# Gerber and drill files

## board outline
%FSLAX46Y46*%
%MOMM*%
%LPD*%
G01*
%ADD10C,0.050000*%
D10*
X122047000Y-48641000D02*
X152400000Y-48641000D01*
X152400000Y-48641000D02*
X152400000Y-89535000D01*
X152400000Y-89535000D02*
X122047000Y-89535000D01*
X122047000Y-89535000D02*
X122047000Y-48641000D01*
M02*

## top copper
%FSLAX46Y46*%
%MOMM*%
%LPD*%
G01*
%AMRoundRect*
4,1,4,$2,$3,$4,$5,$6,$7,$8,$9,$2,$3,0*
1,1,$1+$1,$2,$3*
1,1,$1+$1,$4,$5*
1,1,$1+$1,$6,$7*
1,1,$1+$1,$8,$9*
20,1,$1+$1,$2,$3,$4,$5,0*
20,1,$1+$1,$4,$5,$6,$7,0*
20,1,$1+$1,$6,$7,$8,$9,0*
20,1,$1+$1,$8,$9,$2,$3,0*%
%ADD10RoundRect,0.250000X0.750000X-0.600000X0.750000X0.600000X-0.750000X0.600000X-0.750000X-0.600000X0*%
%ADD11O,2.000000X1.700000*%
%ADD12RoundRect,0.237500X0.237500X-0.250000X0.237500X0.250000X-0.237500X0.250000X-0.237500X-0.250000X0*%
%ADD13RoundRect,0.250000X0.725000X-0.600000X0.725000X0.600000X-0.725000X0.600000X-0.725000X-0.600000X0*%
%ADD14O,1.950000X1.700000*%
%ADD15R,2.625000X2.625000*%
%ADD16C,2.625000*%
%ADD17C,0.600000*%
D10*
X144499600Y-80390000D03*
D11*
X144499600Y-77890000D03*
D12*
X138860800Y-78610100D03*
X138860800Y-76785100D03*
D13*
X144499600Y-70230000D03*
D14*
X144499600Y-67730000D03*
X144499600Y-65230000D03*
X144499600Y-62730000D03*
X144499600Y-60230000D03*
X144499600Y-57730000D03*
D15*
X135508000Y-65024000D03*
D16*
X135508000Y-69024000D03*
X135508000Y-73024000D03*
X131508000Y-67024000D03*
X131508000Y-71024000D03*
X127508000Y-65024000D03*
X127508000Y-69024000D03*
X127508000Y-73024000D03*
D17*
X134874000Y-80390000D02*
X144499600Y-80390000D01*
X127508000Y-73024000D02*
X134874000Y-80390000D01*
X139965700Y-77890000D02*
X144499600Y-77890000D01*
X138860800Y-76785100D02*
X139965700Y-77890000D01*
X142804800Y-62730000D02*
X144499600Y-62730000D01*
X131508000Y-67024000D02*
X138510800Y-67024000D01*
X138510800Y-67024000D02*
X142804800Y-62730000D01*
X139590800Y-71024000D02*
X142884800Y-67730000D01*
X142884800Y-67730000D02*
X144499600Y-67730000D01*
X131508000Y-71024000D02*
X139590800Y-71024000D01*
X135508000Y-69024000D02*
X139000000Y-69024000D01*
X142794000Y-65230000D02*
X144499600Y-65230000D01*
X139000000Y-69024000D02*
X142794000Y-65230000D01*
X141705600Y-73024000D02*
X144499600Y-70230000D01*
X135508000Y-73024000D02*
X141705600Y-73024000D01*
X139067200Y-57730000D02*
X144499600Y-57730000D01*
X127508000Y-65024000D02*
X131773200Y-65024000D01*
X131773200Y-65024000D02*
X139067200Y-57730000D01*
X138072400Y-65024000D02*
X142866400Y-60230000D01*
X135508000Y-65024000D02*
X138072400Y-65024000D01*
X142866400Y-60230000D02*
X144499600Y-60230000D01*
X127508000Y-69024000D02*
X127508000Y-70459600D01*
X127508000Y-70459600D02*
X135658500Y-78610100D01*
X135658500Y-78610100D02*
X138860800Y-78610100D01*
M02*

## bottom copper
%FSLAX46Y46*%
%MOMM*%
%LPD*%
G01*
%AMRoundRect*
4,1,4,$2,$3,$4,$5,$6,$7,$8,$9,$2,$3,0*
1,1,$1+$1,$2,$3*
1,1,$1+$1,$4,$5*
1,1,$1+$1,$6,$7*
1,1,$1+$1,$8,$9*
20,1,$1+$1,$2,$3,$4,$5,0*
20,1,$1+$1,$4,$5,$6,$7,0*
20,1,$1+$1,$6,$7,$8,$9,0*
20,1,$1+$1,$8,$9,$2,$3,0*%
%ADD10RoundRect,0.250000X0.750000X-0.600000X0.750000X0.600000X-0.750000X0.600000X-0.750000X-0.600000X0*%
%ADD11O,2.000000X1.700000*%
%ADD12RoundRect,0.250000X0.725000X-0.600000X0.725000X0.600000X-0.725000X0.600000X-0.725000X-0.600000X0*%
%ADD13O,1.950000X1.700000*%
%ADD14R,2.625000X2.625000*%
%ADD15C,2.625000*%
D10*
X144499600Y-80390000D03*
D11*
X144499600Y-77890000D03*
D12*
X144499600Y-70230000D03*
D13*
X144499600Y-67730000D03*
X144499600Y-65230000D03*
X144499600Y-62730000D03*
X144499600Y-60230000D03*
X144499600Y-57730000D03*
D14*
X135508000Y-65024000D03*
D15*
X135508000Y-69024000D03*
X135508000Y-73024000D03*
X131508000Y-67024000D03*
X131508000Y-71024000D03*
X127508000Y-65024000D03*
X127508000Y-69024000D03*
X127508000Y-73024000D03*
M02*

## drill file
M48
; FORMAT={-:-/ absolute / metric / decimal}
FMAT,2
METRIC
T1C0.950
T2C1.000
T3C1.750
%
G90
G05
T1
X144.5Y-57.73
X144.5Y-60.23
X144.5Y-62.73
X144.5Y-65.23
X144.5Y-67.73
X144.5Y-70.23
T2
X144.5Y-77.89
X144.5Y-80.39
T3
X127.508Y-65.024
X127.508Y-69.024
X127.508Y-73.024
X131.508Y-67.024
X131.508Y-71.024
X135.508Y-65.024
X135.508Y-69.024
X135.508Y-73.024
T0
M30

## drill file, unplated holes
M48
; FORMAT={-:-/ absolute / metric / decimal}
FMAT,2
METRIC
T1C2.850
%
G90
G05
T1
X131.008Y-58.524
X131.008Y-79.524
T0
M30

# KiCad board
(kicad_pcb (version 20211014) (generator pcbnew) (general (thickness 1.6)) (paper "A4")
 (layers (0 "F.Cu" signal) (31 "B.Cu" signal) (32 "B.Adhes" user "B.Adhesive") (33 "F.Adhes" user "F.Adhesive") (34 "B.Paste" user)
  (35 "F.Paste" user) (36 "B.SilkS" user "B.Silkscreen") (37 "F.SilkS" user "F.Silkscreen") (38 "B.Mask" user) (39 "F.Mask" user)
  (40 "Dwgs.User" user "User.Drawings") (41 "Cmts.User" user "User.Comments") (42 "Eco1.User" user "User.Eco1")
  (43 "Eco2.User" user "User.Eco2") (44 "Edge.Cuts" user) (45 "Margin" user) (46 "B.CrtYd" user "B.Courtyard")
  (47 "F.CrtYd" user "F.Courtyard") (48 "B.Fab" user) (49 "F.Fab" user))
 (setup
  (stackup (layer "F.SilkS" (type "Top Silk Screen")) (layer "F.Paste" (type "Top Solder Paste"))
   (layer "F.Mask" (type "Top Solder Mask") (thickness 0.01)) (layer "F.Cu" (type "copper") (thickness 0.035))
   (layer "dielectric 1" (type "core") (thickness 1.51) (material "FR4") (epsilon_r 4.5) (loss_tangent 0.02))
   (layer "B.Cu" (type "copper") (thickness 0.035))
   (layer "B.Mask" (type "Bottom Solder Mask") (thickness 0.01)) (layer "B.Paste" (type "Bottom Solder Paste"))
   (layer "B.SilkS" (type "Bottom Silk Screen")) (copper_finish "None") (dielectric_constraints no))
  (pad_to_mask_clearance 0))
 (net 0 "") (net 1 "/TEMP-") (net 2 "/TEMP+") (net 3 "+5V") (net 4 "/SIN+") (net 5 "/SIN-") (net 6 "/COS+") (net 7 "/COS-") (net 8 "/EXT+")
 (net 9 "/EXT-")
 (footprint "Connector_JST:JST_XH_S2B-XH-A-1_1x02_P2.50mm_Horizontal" (layer "F.Cu") (at 144.4996 80.39 90)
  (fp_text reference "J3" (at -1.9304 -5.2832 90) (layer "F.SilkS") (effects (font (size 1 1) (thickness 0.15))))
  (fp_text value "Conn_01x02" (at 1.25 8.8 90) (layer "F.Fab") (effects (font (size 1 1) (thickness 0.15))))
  (pad "1" thru_hole roundrect (at 0 0 90) (size 1.7 2) (drill 1) (layers *.Cu *.Mask) (roundrect_rratio 0.1470588235) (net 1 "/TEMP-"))
  (pad "2" thru_hole oval (at 2.5 0 90) (size 1.7 2) (drill 1) (layers *.Cu *.Mask) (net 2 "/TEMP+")))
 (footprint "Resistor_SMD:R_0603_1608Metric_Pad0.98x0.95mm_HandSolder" (layer "F.Cu") (at 138.8608 77.6976 90)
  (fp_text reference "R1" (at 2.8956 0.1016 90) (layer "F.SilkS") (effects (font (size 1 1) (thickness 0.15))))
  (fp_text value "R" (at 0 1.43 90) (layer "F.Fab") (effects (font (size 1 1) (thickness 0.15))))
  (pad "1" smd roundrect (at -0.9125 0 90) (size 0.975 0.95) (layers "F.Cu" "F.Paste" "F.Mask") (roundrect_rratio 0.25) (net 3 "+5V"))
  (pad "2" smd roundrect (at 0.9125 0 90) (size 0.975 0.95) (layers "F.Cu" "F.Paste" "F.Mask") (roundrect_rratio 0.25) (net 2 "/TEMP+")))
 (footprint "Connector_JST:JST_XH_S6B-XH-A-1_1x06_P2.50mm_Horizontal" (layer "F.Cu") (at 144.4996 70.23 90)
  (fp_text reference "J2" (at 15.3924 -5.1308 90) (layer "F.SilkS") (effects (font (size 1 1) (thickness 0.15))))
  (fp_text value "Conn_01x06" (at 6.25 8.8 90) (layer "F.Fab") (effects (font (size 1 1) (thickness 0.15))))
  (pad "1" thru_hole roundrect (at 0 0 90) (size 1.7 1.95) (drill 0.95) (layers *.Cu *.Mask) (roundrect_rratio 0.1470588235) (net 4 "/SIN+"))
  (pad "2" thru_hole oval (at 2.5 0 90) (size 1.7 1.95) (drill 0.95) (layers *.Cu *.Mask) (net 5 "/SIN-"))
  (pad "3" thru_hole oval (at 5 0 90) (size 1.7 1.95) (drill 0.95) (layers *.Cu *.Mask) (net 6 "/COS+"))
  (pad "4" thru_hole oval (at 7.5 0 90) (size 1.7 1.95) (drill 0.95) (layers *.Cu *.Mask) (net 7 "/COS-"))
  (pad "5" thru_hole oval (at 10 0 90) (size 1.7 1.95) (drill 0.95) (layers *.Cu *.Mask) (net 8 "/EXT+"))
  (pad "6" thru_hole oval (at 12.5 0 90) (size 1.7 1.95) (drill 0.95) (layers *.Cu *.Mask) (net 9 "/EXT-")))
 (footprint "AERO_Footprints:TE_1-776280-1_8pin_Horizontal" (layer "F.Cu") (at 131.008 69.024 -90)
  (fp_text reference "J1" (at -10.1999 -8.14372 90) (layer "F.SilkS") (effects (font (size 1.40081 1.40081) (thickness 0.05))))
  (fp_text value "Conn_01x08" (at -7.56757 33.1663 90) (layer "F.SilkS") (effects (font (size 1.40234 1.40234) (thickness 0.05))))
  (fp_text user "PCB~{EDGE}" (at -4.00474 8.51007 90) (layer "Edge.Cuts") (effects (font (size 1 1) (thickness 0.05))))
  (pad "" np_thru_hole circle (at -10.5 0 270) (size 2.85 2.85) (drill 2.85) (layers *.Cu *.Mask "F.SilkS"))
  (pad "" np_thru_hole circle (at 10.5 0 270) (size 2.85 2.85) (drill 2.85) (layers *.Cu *.Mask "F.SilkS"))
  (pad "1" thru_hole rect (at -4 -4.5 270) (size 2.625 2.625) (drill 1.75) (layers *.Cu *.Mask) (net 8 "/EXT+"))
  (pad "2" thru_hole circle (at 0 -4.5 270) (size 2.625 2.625) (drill 1.75) (layers *.Cu *.Mask) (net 6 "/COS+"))
  (pad "3" thru_hole circle (at 4 -4.5 270) (size 2.625 2.625) (drill 1.75) (layers *.Cu *.Mask) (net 4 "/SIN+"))
  (pad "4" thru_hole circle (at -2 -0.5 270) (size 2.625 2.625) (drill 1.75) (layers *.Cu *.Mask) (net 7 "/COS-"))
  (pad "5" thru_hole circle (at 2 -0.5 270) (size 2.625 2.625) (drill 1.75) (layers *.Cu *.Mask) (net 5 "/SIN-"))
  (pad "6" thru_hole circle (at -4 3.5 270) (size 2.625 2.625) (drill 1.75) (layers *.Cu *.Mask) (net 9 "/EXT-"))
  (pad "7" thru_hole circle (at 0 3.5 270) (size 2.625 2.625) (drill 1.75) (layers *.Cu *.Mask) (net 3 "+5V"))
  (pad "8" thru_hole circle (at 4 3.5 270) (size 2.625 2.625) (drill 1.75) (layers *.Cu *.Mask) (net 1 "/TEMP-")))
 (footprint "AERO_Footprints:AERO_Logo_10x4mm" (layer "F.Cu") (at 145.415 86.487)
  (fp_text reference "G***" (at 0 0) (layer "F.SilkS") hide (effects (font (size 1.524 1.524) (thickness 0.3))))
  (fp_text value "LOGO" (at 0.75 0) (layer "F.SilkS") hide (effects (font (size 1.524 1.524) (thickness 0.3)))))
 (gr_rect (start 122.047 48.641) (end 152.4 89.535) (layer "Edge.Cuts") (width 0.05) (fill none))
 (segment (start 134.874 80.39) (end 144.4996 80.39) (width 0.6) (layer "F.Cu") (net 1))
 (segment (start 127.508 73.024) (end 134.874 80.39) (width 0.6) (layer "F.Cu") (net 1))
 (segment (start 139.9657 77.89) (end 144.4996 77.89) (width 0.6) (layer "F.Cu") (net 2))
 (segment (start 138.8608 76.7851) (end 139.9657 77.89) (width 0.6) (layer "F.Cu") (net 2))
 (segment (start 142.8048 62.73) (end 144.4996 62.73) (width 0.6) (layer "F.Cu") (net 7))
 (segment (start 131.508 67.024) (end 138.5108 67.024) (width 0.6) (layer "F.Cu") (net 7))
 (segment (start 138.5108 67.024) (end 142.8048 62.73) (width 0.6) (layer "F.Cu") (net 7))
 (segment (start 139.5908 71.024) (end 142.8848 67.73) (width 0.6) (layer "F.Cu") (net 5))
 (segment (start 142.8848 67.73) (end 144.4996 67.73) (width 0.6) (layer "F.Cu") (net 5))
 (segment (start 131.508 71.024) (end 139.5908 71.024) (width 0.6) (layer "F.Cu") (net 5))
 (segment (start 135.508 69.024) (end 139 69.024) (width 0.6) (layer "F.Cu") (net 6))
 (segment (start 142.794 65.23) (end 144.4996 65.23) (width 0.6) (layer "F.Cu") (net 6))
 (segment (start 139 69.024) (end 142.794 65.23) (width 0.6) (layer "F.Cu") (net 6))
 (segment (start 141.7056 73.024) (end 144.4996 70.23) (width 0.6) (layer "F.Cu") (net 4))
 (segment (start 135.508 73.024) (end 141.7056 73.024) (width 0.6) (layer "F.Cu") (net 4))
 (segment (start 139.0672 57.73) (end 144.4996 57.73) (width 0.6) (layer "F.Cu") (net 9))
 (segment (start 127.508 65.024) (end 131.7732 65.024) (width 0.6) (layer "F.Cu") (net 9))
 (segment (start 131.7732 65.024) (end 139.0672 57.73) (width 0.6) (layer "F.Cu") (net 9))
 (segment (start 138.0724 65.024) (end 142.8664 60.23) (width 0.6) (layer "F.Cu") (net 8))
 (segment (start 135.508 65.024) (end 138.0724 65.024) (width 0.6) (layer "F.Cu") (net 8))
 (segment (start 142.8664 60.23) (end 144.4996 60.23) (width 0.6) (layer "F.Cu") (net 8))
 (segment (start 127.508 69.024) (end 127.508 70.4596) (width 0.6) (layer "F.Cu") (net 3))
 (segment (start 127.508 70.4596) (end 135.6585 78.6101) (width 0.6) (layer "F.Cu") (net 3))
 (segment (start 135.6585 78.6101) (end 138.8608 78.6101) (width 0.6) (layer "F.Cu") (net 3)))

